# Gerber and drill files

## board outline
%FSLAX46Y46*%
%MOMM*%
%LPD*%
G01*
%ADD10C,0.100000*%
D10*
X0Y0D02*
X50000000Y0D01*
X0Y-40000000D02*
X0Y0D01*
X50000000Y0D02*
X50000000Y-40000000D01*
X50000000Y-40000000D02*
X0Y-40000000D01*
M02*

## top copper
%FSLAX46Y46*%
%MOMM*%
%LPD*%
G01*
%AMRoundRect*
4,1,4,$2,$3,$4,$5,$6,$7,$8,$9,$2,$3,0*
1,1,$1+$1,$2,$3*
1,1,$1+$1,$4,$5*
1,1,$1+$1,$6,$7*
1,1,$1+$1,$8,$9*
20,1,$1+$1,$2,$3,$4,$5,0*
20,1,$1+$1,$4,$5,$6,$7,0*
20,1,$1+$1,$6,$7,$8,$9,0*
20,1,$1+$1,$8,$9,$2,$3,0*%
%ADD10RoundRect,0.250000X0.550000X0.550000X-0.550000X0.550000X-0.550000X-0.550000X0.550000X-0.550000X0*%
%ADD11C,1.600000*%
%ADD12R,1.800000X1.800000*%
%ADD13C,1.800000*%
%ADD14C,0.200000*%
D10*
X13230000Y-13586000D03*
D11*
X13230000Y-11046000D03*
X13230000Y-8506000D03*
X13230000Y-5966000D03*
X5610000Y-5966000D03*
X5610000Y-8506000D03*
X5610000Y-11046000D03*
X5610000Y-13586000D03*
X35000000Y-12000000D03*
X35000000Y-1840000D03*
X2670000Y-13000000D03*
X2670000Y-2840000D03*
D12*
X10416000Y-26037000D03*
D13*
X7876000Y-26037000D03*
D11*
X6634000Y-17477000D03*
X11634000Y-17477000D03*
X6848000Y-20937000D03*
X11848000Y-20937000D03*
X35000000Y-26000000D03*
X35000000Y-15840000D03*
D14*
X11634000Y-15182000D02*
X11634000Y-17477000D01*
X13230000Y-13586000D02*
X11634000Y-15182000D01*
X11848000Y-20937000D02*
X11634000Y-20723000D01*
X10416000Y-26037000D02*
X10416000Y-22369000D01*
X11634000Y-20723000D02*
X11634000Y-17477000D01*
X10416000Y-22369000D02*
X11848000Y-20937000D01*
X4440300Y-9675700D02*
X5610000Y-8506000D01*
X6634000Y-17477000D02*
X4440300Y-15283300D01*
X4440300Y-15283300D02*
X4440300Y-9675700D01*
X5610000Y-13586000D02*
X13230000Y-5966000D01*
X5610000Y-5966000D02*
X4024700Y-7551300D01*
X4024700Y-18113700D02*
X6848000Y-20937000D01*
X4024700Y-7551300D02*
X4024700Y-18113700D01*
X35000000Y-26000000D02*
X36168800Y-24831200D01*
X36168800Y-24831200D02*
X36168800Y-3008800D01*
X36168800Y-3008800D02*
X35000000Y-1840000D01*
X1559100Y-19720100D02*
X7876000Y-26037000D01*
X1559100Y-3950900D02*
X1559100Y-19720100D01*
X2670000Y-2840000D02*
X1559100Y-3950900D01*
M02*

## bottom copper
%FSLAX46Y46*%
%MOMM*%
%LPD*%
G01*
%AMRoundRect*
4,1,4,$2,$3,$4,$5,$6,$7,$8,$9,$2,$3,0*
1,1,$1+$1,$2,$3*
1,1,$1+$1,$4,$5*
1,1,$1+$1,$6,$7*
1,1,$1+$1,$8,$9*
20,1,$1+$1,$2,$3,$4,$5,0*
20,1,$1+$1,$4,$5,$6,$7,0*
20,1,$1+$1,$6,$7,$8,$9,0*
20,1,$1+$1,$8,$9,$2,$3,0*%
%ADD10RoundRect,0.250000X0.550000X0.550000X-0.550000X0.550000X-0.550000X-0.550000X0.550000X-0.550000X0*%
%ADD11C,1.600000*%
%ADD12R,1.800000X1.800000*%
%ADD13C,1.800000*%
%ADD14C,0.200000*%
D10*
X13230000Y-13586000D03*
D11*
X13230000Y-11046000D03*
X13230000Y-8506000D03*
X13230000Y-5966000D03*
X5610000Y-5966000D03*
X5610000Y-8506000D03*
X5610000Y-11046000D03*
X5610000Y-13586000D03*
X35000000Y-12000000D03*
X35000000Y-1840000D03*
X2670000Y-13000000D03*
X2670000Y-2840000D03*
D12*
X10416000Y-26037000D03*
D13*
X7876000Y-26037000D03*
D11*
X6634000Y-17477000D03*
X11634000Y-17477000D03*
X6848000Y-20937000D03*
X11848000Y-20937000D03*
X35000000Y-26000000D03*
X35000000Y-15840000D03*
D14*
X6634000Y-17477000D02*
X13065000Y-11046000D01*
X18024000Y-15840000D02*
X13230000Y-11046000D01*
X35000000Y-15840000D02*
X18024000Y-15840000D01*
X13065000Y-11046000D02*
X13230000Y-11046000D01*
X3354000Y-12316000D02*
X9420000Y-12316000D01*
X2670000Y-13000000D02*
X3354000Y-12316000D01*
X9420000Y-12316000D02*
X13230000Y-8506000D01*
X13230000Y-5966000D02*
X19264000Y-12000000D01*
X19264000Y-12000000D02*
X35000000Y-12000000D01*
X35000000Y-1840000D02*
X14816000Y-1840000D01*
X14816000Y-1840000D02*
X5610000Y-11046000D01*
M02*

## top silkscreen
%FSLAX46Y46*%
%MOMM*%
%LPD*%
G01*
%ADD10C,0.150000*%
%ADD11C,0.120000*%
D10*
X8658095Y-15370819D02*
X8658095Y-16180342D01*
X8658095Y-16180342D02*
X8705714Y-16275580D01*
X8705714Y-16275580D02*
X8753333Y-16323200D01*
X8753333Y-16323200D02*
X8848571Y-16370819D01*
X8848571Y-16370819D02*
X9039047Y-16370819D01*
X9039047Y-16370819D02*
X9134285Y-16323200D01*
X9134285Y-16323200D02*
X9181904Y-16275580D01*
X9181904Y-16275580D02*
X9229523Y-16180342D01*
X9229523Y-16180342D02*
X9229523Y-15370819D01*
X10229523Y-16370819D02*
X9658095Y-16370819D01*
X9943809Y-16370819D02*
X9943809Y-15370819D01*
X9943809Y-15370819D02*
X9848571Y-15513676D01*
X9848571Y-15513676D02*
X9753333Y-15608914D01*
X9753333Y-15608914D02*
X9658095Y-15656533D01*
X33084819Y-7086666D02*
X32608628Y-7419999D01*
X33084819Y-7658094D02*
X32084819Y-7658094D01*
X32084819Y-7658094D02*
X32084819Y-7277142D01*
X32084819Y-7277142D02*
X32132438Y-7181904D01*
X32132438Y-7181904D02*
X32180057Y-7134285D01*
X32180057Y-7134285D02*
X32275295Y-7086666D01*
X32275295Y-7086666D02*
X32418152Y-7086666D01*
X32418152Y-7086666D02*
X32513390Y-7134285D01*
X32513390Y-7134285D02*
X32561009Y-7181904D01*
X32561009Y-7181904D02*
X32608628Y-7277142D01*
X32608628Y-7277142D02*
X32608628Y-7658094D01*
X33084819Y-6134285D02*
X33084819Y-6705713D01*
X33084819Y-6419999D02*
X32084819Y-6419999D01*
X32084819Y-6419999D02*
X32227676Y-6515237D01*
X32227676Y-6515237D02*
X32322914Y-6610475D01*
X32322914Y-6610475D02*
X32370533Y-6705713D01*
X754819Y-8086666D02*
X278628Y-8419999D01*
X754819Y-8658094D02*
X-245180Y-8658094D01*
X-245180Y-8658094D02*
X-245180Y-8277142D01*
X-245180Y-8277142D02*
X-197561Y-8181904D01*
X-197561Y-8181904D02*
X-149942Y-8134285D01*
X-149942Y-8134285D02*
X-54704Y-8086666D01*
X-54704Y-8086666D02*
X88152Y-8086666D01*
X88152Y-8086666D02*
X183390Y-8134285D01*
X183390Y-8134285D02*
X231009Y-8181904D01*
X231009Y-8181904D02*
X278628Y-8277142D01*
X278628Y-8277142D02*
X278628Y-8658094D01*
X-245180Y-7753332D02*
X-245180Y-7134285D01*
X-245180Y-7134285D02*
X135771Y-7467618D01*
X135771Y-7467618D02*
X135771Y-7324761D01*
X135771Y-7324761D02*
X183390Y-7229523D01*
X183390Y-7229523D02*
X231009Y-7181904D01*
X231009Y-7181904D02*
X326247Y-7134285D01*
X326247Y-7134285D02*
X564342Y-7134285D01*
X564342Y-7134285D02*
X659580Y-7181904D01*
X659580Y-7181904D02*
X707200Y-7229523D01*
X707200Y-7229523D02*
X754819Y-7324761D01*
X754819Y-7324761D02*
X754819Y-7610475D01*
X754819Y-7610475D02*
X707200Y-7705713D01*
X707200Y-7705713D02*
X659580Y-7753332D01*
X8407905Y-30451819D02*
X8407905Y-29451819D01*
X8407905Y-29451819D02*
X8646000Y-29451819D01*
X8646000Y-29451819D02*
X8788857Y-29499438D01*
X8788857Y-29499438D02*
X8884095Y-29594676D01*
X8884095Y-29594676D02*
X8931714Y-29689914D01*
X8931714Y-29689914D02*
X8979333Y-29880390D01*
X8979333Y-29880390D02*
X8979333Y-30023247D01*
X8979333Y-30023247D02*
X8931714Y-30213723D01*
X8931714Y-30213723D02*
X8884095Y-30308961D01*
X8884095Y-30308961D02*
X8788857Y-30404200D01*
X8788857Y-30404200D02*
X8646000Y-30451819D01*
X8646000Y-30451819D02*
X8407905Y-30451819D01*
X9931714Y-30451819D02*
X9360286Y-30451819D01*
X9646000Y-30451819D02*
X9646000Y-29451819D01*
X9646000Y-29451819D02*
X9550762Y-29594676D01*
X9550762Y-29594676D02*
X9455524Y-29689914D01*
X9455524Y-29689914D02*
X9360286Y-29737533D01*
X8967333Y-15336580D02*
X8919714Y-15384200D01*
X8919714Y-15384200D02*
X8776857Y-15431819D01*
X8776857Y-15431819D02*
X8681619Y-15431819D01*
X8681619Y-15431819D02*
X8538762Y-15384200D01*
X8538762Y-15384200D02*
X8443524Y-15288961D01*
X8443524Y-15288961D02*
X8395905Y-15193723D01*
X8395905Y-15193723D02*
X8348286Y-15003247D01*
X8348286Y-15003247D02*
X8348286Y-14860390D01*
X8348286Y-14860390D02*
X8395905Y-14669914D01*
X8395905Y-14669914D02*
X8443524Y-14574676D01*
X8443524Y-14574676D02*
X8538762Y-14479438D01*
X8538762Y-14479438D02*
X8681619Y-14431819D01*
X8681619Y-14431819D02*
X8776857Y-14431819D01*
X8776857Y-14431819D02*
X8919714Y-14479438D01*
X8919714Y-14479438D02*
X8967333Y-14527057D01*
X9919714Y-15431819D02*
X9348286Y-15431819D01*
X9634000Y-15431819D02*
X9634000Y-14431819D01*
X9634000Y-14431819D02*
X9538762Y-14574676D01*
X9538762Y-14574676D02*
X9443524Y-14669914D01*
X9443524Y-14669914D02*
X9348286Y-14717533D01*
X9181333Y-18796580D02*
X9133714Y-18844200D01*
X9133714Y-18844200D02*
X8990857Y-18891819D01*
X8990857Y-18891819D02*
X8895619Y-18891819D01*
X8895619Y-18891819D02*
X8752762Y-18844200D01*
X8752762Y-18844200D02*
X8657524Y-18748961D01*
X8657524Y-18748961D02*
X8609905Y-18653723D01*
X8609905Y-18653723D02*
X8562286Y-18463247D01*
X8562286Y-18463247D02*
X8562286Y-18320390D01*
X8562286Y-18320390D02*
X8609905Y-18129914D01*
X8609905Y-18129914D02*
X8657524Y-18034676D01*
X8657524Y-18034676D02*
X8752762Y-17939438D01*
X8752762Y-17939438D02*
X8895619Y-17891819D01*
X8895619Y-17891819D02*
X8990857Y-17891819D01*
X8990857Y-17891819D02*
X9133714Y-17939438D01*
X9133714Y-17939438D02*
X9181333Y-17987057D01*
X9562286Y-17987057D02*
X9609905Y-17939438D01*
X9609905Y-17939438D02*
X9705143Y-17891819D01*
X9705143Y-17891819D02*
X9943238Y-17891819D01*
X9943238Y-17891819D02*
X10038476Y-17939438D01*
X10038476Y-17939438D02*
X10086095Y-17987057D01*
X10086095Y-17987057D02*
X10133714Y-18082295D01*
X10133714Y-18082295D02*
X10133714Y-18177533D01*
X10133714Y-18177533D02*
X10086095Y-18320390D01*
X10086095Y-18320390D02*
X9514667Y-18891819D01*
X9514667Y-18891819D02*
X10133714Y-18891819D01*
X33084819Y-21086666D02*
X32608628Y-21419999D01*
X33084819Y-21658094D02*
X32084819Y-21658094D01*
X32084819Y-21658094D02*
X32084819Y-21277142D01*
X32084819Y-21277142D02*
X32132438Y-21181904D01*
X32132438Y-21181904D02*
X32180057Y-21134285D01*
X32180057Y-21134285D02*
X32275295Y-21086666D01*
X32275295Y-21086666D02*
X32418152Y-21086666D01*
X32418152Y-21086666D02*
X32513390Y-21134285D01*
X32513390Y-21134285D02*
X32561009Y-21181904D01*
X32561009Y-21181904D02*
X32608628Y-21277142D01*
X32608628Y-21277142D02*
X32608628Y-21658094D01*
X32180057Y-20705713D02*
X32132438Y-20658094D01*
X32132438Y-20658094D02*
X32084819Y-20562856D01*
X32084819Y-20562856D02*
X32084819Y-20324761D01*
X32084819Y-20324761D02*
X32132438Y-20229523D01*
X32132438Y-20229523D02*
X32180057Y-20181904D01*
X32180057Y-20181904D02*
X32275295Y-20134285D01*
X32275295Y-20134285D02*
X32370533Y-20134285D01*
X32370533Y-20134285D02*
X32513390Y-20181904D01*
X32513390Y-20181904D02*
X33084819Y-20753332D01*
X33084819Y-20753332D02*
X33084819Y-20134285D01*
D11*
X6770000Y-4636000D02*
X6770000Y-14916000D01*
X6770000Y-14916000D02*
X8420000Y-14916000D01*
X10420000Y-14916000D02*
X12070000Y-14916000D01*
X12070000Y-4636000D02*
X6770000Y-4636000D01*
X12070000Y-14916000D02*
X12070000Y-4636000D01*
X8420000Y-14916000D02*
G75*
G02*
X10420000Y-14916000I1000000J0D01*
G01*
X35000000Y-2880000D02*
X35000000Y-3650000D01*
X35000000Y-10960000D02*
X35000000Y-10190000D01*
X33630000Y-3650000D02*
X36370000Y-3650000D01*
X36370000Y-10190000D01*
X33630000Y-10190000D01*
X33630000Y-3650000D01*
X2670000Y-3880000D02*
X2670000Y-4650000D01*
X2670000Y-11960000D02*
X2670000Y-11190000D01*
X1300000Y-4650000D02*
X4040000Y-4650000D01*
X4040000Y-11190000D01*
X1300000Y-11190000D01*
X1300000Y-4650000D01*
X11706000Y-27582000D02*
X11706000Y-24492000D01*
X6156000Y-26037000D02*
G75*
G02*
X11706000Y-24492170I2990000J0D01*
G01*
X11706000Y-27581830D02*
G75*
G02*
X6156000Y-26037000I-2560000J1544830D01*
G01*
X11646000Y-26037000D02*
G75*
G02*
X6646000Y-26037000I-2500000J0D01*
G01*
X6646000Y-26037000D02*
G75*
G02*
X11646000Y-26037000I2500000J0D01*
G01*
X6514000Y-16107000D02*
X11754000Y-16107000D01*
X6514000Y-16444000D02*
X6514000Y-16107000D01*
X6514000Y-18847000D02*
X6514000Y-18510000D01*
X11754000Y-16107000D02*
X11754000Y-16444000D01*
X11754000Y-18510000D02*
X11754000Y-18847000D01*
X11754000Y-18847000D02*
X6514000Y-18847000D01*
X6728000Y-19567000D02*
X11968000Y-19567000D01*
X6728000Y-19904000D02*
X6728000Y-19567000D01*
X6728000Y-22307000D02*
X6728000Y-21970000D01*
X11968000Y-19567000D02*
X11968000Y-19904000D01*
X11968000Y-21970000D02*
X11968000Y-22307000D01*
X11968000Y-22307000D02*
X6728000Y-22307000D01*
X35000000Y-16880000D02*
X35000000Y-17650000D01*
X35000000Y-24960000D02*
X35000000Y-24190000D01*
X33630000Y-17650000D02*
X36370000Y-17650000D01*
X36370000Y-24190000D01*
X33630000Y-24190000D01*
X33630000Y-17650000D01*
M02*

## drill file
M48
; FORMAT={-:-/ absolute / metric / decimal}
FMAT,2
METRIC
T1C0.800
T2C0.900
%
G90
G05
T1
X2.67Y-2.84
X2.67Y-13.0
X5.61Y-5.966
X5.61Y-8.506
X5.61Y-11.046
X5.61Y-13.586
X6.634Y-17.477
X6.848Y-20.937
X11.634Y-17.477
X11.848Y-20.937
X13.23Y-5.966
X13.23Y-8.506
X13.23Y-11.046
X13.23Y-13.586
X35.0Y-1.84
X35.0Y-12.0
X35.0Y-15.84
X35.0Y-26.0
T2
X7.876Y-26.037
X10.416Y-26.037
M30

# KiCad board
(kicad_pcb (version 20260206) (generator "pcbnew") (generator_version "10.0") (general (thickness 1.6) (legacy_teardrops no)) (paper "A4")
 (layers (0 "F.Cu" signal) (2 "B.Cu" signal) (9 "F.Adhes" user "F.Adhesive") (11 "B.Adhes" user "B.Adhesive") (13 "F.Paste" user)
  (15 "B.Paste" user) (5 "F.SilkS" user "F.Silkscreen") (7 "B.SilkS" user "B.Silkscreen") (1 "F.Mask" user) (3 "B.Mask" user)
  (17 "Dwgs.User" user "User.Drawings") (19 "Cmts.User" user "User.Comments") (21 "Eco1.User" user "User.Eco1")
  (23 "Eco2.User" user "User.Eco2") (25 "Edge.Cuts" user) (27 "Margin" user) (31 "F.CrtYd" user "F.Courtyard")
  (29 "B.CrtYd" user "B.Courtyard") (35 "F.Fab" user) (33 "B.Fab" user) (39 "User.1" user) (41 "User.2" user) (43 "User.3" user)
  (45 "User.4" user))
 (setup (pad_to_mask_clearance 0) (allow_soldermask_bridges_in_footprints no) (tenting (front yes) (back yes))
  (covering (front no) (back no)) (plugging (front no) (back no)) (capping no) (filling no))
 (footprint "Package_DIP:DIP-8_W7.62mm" (layer "F.Cu") (at 13.23 13.586 180)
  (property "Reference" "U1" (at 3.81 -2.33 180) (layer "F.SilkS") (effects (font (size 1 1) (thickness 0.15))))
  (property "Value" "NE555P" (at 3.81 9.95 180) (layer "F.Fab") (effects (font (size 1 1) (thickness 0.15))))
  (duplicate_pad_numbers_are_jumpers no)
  (fp_line (start 6.46 8.95) (end 6.46 -1.33) (stroke (width 0.12) (type solid)) (layer "F.SilkS"))
  (fp_line (start 6.46 -1.33) (end 4.81 -1.33) (stroke (width 0.12) (type solid)) (layer "F.SilkS"))
  (fp_line (start 2.81 -1.33) (end 1.16 -1.33) (stroke (width 0.12) (type solid)) (layer "F.SilkS"))
  (fp_line (start 1.16 8.95) (end 6.46 8.95) (stroke (width 0.12) (type solid)) (layer "F.SilkS"))
  (fp_line (start 1.16 -1.33) (end 1.16 8.95) (stroke (width 0.12) (type solid)) (layer "F.SilkS"))
  (fp_arc (start 4.81 -1.33) (mid 3.81 -0.33) (end 2.81 -1.33) (stroke (width 0.12) (type solid)) (layer "F.SilkS"))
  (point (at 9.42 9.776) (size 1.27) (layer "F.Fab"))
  (pad "1" thru_hole roundrect (at 0 0 180) (size 1.6 1.6) (drill 0.8) (layers "*.Cu" "*.Mask") (remove_unused_layers no)
   (roundrect_rratio 0.15625) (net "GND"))
  (pad "2" thru_hole circle (at 0 2.54 180) (size 1.6 1.6) (drill 0.8) (layers "*.Cu" "*.Mask") (remove_unused_layers no) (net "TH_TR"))
  (pad "3" thru_hole circle (at 0 5.08 180) (size 1.6 1.6) (drill 0.8) (layers "*.Cu" "*.Mask") (remove_unused_layers no) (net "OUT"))
  (pad "4" thru_hole circle (at 0 7.62 180) (size 1.6 1.6) (drill 0.8) (layers "*.Cu" "*.Mask") (remove_unused_layers no) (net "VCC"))
  (pad "5" thru_hole circle (at 7.62 7.62 180) (size 1.6 1.6) (drill 0.8) (layers "*.Cu" "*.Mask") (remove_unused_layers no) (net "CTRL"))
  (pad "6" thru_hole circle (at 7.62 5.08 180) (size 1.6 1.6) (drill 0.8) (layers "*.Cu" "*.Mask") (remove_unused_layers no) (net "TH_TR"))
  (pad "7" thru_hole circle (at 7.62 2.54 180) (size 1.6 1.6) (drill 0.8) (layers "*.Cu" "*.Mask") (remove_unused_layers no) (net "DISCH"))
  (pad "8" thru_hole circle (at 7.62 0 180) (size 1.6 1.6) (drill 0.8) (layers "*.Cu" "*.Mask") (remove_unused_layers no) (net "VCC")))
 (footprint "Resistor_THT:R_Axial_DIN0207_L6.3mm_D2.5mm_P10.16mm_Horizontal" (layer "F.Cu") (at 35 12 90)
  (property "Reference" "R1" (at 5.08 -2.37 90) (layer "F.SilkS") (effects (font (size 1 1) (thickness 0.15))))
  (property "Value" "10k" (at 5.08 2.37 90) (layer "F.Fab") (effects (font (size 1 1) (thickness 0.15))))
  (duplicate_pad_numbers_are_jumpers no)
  (fp_line (start 9.12 0) (end 8.35 0) (stroke (width 0.12) (type solid)) (layer "F.SilkS"))
  (fp_line (start 1.04 0) (end 1.81 0) (stroke (width 0.12) (type solid)) (layer "F.SilkS"))
  (fp_rect (start 1.81 -1.37) (end 8.35 1.37) (stroke (width 0.12) (type solid)) (fill no) (layer "F.SilkS"))
  (pad "1" thru_hole circle (at 0 0 90) (size 1.6 1.6) (drill 0.8) (layers "*.Cu" "*.Mask") (remove_unused_layers no) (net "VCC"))
  (pad "2" thru_hole circle (at 10.16 0 90) (size 1.6 1.6) (drill 0.8) (layers "*.Cu" "*.Mask") (remove_unused_layers no) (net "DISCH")))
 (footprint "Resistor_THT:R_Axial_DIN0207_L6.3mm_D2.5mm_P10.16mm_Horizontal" (layer "F.Cu") (at 2.67 13 90)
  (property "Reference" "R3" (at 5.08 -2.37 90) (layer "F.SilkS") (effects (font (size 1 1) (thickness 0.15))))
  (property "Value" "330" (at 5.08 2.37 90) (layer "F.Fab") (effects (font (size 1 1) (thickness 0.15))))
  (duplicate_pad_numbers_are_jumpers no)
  (fp_line (start 9.12 0) (end 8.35 0) (stroke (width 0.12) (type solid)) (layer "F.SilkS"))
  (fp_line (start 1.04 0) (end 1.81 0) (stroke (width 0.12) (type solid)) (layer "F.SilkS"))
  (fp_rect (start 1.81 -1.37) (end 8.35 1.37) (stroke (width 0.12) (type solid)) (fill no) (layer "F.SilkS"))
  (pad "1" thru_hole circle (at 0 0 90) (size 1.6 1.6) (drill 0.8) (layers "*.Cu" "*.Mask") (remove_unused_layers no) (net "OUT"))
  (pad "2" thru_hole circle (at 10.16 0 90) (size 1.6 1.6) (drill 0.8) (layers "*.Cu" "*.Mask") (remove_unused_layers no) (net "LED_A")))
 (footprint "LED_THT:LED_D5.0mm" (layer "F.Cu") (at 10.416 26.037 180)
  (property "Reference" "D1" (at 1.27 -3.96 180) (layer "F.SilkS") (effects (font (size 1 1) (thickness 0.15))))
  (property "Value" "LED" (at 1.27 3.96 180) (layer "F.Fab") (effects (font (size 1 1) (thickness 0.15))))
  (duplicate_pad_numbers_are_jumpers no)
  (fp_line (start -1.29 -1.545) (end -1.29 1.545) (stroke (width 0.12) (type solid)) (layer "F.SilkS"))
  (fp_arc (start 4.26 0) (mid 2.071779 2.880495) (end -1.29 1.54483) (stroke (width 0.12) (type solid)) (layer "F.SilkS"))
  (fp_arc (start -1.29 -1.54483) (mid 2.071779 -2.880495) (end 4.26 0) (stroke (width 0.12) (type solid)) (layer "F.SilkS"))
  (fp_circle (center 1.27 0) (end 3.77 0) (stroke (width 0.12) (type solid)) (fill no) (layer "F.SilkS"))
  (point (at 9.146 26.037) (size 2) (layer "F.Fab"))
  (pad "1" thru_hole rect (at 0 0 180) (size 1.8 1.8) (drill 0.9) (layers "*.Cu" "*.Mask") (remove_unused_layers no) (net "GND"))
  (pad "2" thru_hole circle (at 2.54 0 180) (size 1.8 1.8) (drill 0.9) (layers "*.Cu" "*.Mask") (remove_unused_layers no) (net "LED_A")))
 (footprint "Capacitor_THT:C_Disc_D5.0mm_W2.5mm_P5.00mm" (layer "F.Cu") (at 6.634 17.477)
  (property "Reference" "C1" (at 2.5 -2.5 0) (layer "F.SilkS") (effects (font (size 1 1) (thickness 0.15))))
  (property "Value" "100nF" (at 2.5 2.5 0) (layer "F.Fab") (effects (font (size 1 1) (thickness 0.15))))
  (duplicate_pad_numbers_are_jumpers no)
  (fp_line (start -0.12 -1.37) (end 5.12 -1.37) (stroke (width 0.12) (type solid)) (layer "F.SilkS"))
  (fp_line (start -0.12 -1.033) (end -0.12 -1.37) (stroke (width 0.12) (type solid)) (layer "F.SilkS"))
  (fp_line (start -0.12 1.37) (end -0.12 1.033) (stroke (width 0.12) (type solid)) (layer "F.SilkS"))
  (fp_line (start 5.12 -1.37) (end 5.12 -1.033) (stroke (width 0.12) (type solid)) (layer "F.SilkS"))
  (fp_line (start 5.12 1.033) (end 5.12 1.37) (stroke (width 0.12) (type solid)) (layer "F.SilkS"))
  (fp_line (start 5.12 1.37) (end -0.12 1.37) (stroke (width 0.12) (type solid)) (layer "F.SilkS"))
  (pad "1" thru_hole circle (at 0 0) (size 1.6 1.6) (drill 0.8) (layers "*.Cu" "*.Mask") (remove_unused_layers no) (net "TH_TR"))
  (pad "2" thru_hole circle (at 5 0) (size 1.6 1.6) (drill 0.8) (layers "*.Cu" "*.Mask") (remove_unused_layers no) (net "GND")))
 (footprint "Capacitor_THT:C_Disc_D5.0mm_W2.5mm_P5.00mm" (layer "F.Cu") (at 6.848 20.937)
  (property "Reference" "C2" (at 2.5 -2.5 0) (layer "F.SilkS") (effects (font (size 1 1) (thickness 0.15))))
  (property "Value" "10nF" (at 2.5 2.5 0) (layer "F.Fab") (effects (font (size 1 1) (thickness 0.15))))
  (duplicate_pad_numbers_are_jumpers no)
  (fp_line (start -0.12 -1.37) (end 5.12 -1.37) (stroke (width 0.12) (type solid)) (layer "F.SilkS"))
  (fp_line (start -0.12 -1.033) (end -0.12 -1.37) (stroke (width 0.12) (type solid)) (layer "F.SilkS"))
  (fp_line (start -0.12 1.37) (end -0.12 1.033) (stroke (width 0.12) (type solid)) (layer "F.SilkS"))
  (fp_line (start 5.12 -1.37) (end 5.12 -1.033) (stroke (width 0.12) (type solid)) (layer "F.SilkS"))
  (fp_line (start 5.12 1.033) (end 5.12 1.37) (stroke (width 0.12) (type solid)) (layer "F.SilkS"))
  (fp_line (start 5.12 1.37) (end -0.12 1.37) (stroke (width 0.12) (type solid)) (layer "F.SilkS"))
  (pad "1" thru_hole circle (at 0 0) (size 1.6 1.6) (drill 0.8) (layers "*.Cu" "*.Mask") (remove_unused_layers no) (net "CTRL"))
  (pad "2" thru_hole circle (at 5 0) (size 1.6 1.6) (drill 0.8) (layers "*.Cu" "*.Mask") (remove_unused_layers no) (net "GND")))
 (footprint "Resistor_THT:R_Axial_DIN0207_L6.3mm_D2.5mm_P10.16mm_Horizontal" (layer "F.Cu") (at 35 26 90)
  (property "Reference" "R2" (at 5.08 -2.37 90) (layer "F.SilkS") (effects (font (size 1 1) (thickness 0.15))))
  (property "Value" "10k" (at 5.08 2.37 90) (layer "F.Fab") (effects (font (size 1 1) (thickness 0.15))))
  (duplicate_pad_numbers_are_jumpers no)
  (fp_line (start 9.12 0) (end 8.35 0) (stroke (width 0.12) (type solid)) (layer "F.SilkS"))
  (fp_line (start 1.04 0) (end 1.81 0) (stroke (width 0.12) (type solid)) (layer "F.SilkS"))
  (fp_rect (start 1.81 -1.37) (end 8.35 1.37) (stroke (width 0.12) (type solid)) (fill no) (layer "F.SilkS"))
  (pad "1" thru_hole circle (at 0 0 90) (size 1.6 1.6) (drill 0.8) (layers "*.Cu" "*.Mask") (remove_unused_layers no) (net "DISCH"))
  (pad "2" thru_hole circle (at 10.16 0 90) (size 1.6 1.6) (drill 0.8) (layers "*.Cu" "*.Mask") (remove_unused_layers no) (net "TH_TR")))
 (gr_line (start 0 0) (end 50 0) (stroke (width 0.1) (type default)) (layer "Edge.Cuts"))
 (gr_line (start 0 40) (end 0 0) (stroke (width 0.1) (type default)) (layer "Edge.Cuts"))
 (gr_line (start 50 0) (end 50 40) (stroke (width 0.1) (type default)) (layer "Edge.Cuts"))
 (gr_line (start 50 40) (end 0 40) (stroke (width 0.1) (type default)) (layer "Edge.Cuts"))
 (segment (start 11.634 15.182) (end 11.634 17.477) (width 0.2) (layer "F.Cu") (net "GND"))
 (segment (start 13.23 13.586) (end 11.634 15.182) (width 0.2) (layer "F.Cu") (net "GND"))
 (segment (start 11.848 20.937) (end 11.634 20.723) (width 0.2) (layer "F.Cu") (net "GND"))
 (segment (start 10.416 26.037) (end 10.416 22.369) (width 0.2) (layer "F.Cu") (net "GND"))
 (segment (start 11.634 20.723) (end 11.634 17.477) (width 0.2) (layer "F.Cu") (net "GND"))
 (segment (start 10.416 22.369) (end 11.848 20.937) (width 0.2) (layer "F.Cu") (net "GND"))
 (segment (start 4.4403 9.6757) (end 5.61 8.506) (width 0.2) (layer "F.Cu") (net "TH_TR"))
 (segment (start 6.634 17.477) (end 4.4403 15.2833) (width 0.2) (layer "F.Cu") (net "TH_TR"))
 (segment (start 4.4403 15.2833) (end 4.4403 9.6757) (width 0.2) (layer "F.Cu") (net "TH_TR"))
 (segment (start 6.634 17.477) (end 13.065 11.046) (width 0.2) (layer "B.Cu") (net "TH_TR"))
 (segment (start 18.024 15.84) (end 13.23 11.046) (width 0.2) (layer "B.Cu") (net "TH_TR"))
 (segment (start 35 15.84) (end 18.024 15.84) (width 0.2) (layer "B.Cu") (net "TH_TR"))
 (segment (start 13.065 11.046) (end 13.23 11.046) (width 0.2) (layer "B.Cu") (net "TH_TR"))
 (segment (start 3.354 12.316) (end 9.42 12.316) (width 0.2) (layer "B.Cu") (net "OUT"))
 (segment (start 2.67 13) (end 3.354 12.316) (width 0.2) (layer "B.Cu") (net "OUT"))
 (segment (start 9.42 12.316) (end 13.23 8.506) (width 0.2) (layer "B.Cu") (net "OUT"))
 (segment (start 5.61 13.586) (end 13.23 5.966) (width 0.2) (layer "F.Cu") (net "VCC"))
 (segment (start 13.23 5.966) (end 19.264 12) (width 0.2) (layer "B.Cu") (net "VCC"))
 (segment (start 19.264 12) (end 35 12) (width 0.2) (layer "B.Cu") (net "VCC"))
 (segment (start 5.61 5.966) (end 4.0247 7.5513) (width 0.2) (layer "F.Cu") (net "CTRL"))
 (segment (start 4.0247 18.1137) (end 6.848 20.937) (width 0.2) (layer "F.Cu") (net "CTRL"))
 (segment (start 4.0247 7.5513) (end 4.0247 18.1137) (width 0.2) (layer "F.Cu") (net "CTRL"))
 (segment (start 35 26) (end 36.1688 24.8312) (width 0.2) (layer "F.Cu") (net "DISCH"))
 (segment (start 36.1688 24.8312) (end 36.1688 3.0088) (width 0.2) (layer "F.Cu") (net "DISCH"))
 (segment (start 36.1688 3.0088) (end 35 1.84) (width 0.2) (layer "F.Cu") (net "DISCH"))
 (segment (start 35 1.84) (end 14.816 1.84) (width 0.2) (layer "B.Cu") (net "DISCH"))
 (segment (start 14.816 1.84) (end 5.61 11.046) (width 0.2) (layer "B.Cu") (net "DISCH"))
 (segment (start 1.5591 19.7201) (end 7.876 26.037) (width 0.2) (layer "F.Cu") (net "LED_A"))
 (segment (start 1.5591 3.9509) (end 1.5591 19.7201) (width 0.2) (layer "F.Cu") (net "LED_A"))
 (segment (start 2.67 2.84) (end 1.5591 3.9509) (width 0.2) (layer "F.Cu") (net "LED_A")))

